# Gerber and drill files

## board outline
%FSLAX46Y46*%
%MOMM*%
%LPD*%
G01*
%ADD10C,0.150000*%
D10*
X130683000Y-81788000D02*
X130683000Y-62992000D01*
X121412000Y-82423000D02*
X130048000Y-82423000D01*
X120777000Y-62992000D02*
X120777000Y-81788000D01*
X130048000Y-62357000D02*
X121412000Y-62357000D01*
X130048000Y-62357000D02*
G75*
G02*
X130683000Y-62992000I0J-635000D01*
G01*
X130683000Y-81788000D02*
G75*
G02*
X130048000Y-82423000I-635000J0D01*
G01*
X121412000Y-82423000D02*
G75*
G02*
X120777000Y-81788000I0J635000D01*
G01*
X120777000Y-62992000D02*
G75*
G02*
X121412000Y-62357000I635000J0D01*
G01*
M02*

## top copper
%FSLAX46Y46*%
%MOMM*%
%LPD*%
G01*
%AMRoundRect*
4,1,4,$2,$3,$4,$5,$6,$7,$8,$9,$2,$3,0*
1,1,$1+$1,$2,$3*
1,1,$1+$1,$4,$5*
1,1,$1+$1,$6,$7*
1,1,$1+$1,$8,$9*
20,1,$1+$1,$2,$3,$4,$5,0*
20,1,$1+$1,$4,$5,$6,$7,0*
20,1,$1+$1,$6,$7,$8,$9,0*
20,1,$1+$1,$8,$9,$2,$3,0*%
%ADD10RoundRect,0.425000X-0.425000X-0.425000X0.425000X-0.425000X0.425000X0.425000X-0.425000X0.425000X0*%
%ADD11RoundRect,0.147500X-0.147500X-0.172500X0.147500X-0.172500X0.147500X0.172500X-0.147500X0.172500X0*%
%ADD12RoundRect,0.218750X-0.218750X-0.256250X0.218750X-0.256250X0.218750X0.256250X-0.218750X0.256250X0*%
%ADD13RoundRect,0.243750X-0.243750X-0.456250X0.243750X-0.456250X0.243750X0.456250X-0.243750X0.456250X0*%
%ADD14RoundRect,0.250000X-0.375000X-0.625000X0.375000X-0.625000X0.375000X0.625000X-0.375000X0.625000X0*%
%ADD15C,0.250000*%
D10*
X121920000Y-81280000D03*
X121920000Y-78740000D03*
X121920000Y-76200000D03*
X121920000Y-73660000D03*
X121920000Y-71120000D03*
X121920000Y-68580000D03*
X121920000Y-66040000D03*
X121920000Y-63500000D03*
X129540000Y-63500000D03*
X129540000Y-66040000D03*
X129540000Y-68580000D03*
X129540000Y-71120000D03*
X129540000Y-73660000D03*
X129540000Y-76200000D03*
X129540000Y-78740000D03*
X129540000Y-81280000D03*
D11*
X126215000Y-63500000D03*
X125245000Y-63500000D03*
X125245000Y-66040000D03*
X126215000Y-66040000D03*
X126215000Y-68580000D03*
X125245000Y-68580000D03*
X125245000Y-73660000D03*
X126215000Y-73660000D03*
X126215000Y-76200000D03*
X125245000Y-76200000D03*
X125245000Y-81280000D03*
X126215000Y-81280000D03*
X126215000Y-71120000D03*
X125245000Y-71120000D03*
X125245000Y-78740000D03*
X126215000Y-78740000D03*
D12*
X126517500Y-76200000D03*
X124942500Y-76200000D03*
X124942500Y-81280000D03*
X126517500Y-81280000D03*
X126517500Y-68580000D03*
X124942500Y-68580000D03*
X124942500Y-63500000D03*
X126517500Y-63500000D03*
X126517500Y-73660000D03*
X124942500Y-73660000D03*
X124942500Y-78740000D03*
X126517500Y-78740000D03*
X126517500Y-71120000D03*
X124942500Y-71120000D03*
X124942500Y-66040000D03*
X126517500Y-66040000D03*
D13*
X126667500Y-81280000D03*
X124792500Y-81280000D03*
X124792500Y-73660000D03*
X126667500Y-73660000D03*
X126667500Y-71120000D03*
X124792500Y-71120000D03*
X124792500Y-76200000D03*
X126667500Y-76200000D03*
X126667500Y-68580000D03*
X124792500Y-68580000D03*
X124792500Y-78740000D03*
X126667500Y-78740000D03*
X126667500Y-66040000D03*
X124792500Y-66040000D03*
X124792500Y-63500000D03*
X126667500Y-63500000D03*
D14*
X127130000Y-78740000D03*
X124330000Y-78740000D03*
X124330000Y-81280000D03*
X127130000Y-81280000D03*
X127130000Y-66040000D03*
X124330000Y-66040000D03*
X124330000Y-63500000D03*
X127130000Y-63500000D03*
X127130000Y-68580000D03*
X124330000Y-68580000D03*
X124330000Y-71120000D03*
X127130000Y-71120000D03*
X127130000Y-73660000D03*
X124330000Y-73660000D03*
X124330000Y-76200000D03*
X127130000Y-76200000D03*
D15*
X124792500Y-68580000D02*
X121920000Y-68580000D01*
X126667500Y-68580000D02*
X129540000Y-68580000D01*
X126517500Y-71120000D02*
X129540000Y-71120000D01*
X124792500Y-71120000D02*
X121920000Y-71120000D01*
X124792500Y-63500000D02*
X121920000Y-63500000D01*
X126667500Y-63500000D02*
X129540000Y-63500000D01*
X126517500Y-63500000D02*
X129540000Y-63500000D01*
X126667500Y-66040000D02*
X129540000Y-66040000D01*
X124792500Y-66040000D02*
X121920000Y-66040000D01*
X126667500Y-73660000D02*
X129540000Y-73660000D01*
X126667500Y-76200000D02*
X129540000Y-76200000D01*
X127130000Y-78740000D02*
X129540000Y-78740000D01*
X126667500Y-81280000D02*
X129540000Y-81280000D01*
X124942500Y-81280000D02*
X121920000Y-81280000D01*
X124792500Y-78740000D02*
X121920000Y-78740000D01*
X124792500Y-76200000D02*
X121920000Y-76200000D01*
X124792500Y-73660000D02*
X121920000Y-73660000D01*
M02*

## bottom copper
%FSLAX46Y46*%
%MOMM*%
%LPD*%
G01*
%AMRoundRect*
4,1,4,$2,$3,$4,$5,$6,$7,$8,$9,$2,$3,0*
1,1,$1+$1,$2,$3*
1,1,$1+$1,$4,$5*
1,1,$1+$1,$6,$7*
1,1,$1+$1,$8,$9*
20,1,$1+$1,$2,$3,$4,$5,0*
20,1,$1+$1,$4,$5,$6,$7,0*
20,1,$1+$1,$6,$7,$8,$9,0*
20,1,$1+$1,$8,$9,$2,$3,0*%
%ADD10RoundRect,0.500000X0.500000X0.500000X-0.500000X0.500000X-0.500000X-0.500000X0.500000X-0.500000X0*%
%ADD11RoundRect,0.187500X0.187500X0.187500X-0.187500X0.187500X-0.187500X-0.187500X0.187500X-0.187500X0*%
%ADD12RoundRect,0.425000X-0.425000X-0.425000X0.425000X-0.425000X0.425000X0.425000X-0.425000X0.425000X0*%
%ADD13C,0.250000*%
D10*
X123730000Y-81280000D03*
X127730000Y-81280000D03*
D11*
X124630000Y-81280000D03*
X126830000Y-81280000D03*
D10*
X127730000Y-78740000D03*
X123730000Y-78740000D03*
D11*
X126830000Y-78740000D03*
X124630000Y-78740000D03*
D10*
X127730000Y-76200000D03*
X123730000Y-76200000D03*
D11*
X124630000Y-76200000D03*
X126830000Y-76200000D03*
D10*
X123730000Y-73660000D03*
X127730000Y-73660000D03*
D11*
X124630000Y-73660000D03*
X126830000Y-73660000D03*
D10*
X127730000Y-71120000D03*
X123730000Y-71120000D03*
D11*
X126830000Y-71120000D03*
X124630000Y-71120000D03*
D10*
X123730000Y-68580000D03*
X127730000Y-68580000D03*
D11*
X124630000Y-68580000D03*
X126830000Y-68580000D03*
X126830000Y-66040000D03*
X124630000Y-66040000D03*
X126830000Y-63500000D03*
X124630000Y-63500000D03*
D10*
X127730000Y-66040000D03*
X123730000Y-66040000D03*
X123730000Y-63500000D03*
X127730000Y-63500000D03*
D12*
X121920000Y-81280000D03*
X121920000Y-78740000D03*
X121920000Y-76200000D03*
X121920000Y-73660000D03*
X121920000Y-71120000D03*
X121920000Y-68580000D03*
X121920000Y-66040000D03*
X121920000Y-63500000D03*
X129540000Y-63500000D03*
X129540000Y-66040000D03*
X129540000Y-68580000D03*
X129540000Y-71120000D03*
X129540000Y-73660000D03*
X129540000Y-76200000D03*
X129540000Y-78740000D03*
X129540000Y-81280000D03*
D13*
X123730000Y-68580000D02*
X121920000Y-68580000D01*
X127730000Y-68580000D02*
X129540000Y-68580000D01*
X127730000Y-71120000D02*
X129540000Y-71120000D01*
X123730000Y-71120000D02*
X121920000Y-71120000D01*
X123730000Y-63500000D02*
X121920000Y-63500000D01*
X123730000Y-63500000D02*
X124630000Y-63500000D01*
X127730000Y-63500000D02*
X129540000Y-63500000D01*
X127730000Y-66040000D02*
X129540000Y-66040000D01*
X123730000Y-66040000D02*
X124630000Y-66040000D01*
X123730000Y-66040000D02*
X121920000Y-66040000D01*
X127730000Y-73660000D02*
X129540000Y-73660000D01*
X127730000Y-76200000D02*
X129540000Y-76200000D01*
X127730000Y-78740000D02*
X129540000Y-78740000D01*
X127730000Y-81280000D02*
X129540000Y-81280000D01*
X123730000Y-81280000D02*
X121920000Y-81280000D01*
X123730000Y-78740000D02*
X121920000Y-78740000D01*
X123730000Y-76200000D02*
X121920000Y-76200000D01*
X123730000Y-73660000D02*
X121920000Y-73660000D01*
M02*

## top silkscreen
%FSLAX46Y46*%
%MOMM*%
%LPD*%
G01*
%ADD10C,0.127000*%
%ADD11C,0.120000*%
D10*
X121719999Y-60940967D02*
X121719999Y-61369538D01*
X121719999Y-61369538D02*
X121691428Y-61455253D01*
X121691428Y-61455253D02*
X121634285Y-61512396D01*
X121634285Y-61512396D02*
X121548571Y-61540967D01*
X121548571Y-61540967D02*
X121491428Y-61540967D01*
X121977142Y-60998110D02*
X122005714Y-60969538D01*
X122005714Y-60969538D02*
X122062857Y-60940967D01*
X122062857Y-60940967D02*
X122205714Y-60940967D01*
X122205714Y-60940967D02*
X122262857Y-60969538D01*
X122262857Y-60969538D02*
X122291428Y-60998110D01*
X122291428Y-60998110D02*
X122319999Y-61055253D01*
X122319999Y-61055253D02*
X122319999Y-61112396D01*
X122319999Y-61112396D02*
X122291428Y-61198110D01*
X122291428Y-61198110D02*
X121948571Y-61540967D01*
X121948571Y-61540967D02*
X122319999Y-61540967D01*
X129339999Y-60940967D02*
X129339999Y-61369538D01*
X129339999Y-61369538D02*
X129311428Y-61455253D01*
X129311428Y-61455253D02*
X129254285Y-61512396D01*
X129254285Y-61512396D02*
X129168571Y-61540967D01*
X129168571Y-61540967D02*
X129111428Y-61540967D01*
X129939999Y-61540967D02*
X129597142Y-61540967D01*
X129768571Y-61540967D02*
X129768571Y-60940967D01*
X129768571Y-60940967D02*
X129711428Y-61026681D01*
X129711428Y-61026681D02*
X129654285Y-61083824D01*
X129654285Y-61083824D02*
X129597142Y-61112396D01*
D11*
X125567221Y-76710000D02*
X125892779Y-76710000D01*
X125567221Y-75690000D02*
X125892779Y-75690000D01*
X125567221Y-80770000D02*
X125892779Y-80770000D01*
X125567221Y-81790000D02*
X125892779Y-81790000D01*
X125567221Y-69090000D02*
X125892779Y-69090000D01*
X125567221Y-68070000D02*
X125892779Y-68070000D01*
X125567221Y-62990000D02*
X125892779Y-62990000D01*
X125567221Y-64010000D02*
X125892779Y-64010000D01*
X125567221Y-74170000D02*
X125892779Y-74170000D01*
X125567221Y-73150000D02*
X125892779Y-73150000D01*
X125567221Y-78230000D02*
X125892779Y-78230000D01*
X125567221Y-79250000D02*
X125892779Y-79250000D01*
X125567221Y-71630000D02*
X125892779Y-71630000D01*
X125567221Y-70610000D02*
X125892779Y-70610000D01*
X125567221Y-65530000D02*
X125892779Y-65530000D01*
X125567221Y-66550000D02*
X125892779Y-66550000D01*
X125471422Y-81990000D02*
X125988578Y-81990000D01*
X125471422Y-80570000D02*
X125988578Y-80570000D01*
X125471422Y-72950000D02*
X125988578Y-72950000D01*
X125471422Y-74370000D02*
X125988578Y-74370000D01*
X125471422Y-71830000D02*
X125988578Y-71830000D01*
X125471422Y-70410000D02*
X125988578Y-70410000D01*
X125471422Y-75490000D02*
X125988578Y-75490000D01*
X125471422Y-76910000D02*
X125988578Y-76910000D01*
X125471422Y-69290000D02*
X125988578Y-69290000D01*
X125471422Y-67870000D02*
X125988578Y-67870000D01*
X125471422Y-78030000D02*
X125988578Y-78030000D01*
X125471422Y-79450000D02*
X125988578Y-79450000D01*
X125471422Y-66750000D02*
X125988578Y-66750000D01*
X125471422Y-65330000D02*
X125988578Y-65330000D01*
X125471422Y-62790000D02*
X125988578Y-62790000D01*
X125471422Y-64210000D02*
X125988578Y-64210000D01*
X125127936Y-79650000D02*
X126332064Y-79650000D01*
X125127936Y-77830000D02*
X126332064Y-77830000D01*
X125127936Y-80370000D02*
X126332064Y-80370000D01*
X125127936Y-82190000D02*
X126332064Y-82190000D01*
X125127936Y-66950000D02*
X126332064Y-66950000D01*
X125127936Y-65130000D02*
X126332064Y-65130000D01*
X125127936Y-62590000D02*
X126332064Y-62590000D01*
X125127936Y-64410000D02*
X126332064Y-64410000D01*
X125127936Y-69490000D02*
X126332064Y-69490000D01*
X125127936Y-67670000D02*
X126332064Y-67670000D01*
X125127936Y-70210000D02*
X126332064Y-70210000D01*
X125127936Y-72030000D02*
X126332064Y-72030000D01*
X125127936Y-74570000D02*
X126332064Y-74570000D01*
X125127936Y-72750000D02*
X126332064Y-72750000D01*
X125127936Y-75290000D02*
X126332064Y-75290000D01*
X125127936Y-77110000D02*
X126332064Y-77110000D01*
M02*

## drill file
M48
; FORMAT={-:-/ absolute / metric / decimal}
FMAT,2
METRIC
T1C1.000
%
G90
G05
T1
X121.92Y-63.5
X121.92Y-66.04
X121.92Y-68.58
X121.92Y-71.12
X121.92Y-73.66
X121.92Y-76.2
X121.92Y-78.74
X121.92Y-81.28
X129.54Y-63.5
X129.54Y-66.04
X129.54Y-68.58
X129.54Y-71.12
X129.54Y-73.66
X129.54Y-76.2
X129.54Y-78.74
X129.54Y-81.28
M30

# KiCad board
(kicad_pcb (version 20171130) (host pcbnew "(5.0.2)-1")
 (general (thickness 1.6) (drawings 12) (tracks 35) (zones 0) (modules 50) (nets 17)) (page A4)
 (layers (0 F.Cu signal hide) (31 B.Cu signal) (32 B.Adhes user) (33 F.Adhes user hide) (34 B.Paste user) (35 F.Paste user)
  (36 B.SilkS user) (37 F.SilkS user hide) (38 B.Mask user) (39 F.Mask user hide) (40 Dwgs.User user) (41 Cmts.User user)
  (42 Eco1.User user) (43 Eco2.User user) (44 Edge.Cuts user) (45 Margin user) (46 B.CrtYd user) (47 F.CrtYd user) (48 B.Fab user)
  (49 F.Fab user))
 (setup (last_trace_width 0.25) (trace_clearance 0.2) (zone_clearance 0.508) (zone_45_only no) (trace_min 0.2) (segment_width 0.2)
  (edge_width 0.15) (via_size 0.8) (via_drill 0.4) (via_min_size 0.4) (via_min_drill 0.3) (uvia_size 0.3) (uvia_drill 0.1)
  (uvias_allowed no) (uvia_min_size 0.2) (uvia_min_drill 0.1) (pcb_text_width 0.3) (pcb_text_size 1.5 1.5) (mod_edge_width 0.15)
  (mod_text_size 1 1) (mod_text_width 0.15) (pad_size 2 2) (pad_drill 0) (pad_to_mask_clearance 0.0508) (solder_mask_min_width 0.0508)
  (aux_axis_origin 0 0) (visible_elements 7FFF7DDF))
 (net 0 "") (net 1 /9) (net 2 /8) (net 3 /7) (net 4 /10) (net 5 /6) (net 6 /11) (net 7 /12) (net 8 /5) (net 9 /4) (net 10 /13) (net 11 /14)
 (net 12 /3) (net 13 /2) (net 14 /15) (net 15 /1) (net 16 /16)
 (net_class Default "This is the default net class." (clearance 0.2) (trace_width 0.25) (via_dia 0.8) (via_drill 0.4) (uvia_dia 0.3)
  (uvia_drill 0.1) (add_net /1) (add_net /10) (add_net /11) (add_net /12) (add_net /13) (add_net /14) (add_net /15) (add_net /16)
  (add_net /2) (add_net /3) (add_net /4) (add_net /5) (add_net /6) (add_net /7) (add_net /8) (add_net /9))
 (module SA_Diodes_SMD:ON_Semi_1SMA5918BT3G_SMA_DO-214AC (layer B.Cu) (at 125.73 81.28 180)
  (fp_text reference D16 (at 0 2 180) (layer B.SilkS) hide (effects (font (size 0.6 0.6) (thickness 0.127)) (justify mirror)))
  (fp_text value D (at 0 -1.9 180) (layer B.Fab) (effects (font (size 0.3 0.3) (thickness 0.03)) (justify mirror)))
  (pad 2 smd roundrect (at 2 0 180) (size 2 2) (layers B.Cu B.Paste B.Mask) (roundrect_rratio 0.25) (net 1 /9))
  (pad 1 smd roundrect (at -2 0 180) (size 2 2) (layers B.Cu B.Paste B.Mask) (roundrect_rratio 0.25) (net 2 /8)))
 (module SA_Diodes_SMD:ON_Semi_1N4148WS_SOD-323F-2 (layer B.Cu) (at 125.73 81.28 180)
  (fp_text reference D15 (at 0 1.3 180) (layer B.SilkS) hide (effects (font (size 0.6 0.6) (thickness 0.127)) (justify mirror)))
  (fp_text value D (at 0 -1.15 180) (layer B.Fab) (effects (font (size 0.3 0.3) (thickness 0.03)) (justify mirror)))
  (pad 2 smd roundrect (at 1.1 0 180) (size 0.75 0.75) (layers B.Cu B.Paste B.Mask) (roundrect_rratio 0.25) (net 1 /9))
  (pad 1 smd roundrect (at -1.1 0 180) (size 0.75 0.75) (layers B.Cu B.Paste B.Mask) (roundrect_rratio 0.25) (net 2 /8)))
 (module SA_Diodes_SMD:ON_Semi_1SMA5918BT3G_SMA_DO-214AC (layer B.Cu) (at 125.73 78.74 180)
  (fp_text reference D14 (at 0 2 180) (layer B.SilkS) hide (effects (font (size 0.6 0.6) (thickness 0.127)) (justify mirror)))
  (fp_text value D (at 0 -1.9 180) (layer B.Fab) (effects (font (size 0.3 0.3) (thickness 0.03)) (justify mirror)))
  (pad 1 smd roundrect (at -2 0 180) (size 2 2) (layers B.Cu B.Paste B.Mask) (roundrect_rratio 0.25) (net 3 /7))
  (pad 2 smd roundrect (at 2 0 180) (size 2 2) (layers B.Cu B.Paste B.Mask) (roundrect_rratio 0.25) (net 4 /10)))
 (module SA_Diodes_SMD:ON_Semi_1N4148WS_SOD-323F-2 (layer B.Cu) (at 125.73 78.74 180)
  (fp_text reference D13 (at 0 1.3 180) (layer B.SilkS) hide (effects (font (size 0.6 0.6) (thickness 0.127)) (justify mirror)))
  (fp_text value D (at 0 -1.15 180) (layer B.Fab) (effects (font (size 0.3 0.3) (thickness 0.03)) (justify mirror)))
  (pad 1 smd roundrect (at -1.1 0 180) (size 0.75 0.75) (layers B.Cu B.Paste B.Mask) (roundrect_rratio 0.25) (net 3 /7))
  (pad 2 smd roundrect (at 1.1 0 180) (size 0.75 0.75) (layers B.Cu B.Paste B.Mask) (roundrect_rratio 0.25) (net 4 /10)))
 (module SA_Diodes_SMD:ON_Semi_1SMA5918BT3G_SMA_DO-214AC (layer B.Cu) (at 125.73 76.2 180)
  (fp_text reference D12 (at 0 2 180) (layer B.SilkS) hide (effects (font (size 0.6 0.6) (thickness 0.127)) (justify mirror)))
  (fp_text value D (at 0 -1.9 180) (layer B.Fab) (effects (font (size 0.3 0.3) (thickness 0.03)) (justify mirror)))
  (pad 1 smd roundrect (at -2 0 180) (size 2 2) (layers B.Cu B.Paste B.Mask) (roundrect_rratio 0.25) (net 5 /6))
  (pad 2 smd roundrect (at 2 0 180) (size 2 2) (layers B.Cu B.Paste B.Mask) (roundrect_rratio 0.25) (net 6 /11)))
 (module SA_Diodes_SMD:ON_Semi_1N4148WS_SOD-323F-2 (layer B.Cu) (at 125.73 76.2 180)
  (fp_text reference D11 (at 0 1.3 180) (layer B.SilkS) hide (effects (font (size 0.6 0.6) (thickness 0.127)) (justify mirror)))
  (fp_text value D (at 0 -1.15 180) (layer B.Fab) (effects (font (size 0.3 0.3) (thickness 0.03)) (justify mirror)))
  (pad 2 smd roundrect (at 1.1 0 180) (size 0.75 0.75) (layers B.Cu B.Paste B.Mask) (roundrect_rratio 0.25) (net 6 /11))
  (pad 1 smd roundrect (at -1.1 0 180) (size 0.75 0.75) (layers B.Cu B.Paste B.Mask) (roundrect_rratio 0.25) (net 5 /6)))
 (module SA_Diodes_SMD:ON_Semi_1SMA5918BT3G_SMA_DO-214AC (layer B.Cu) (at 125.73 73.66 180)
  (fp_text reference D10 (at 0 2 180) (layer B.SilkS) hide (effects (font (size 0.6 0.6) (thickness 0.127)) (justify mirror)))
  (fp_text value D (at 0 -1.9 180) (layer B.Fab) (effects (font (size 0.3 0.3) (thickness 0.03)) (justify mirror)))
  (pad 2 smd roundrect (at 2 0 180) (size 2 2) (layers B.Cu B.Paste B.Mask) (roundrect_rratio 0.25) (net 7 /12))
  (pad 1 smd roundrect (at -2 0 180) (size 2 2) (layers B.Cu B.Paste B.Mask) (roundrect_rratio 0.25) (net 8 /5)))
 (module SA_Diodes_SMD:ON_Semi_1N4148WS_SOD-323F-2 (layer B.Cu) (at 125.73 73.66 180)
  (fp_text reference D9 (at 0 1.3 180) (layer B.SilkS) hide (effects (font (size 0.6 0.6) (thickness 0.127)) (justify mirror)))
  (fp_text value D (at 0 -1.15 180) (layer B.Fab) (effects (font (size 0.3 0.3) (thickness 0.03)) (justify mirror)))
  (pad 2 smd roundrect (at 1.1 0 180) (size 0.75 0.75) (layers B.Cu B.Paste B.Mask) (roundrect_rratio 0.25) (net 7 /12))
  (pad 1 smd roundrect (at -1.1 0 180) (size 0.75 0.75) (layers B.Cu B.Paste B.Mask) (roundrect_rratio 0.25) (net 8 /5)))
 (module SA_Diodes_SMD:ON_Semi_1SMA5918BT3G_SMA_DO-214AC (layer B.Cu) (at 125.73 71.12 180)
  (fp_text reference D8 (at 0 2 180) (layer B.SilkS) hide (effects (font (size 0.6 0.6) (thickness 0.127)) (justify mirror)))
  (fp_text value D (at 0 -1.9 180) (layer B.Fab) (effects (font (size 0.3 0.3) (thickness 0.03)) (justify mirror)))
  (pad 1 smd roundrect (at -2 0 180) (size 2 2) (layers B.Cu B.Paste B.Mask) (roundrect_rratio 0.25) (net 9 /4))
  (pad 2 smd roundrect (at 2 0 180) (size 2 2) (layers B.Cu B.Paste B.Mask) (roundrect_rratio 0.25) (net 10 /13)))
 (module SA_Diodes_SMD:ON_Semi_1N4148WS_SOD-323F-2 (layer B.Cu) (at 125.73 71.12 180)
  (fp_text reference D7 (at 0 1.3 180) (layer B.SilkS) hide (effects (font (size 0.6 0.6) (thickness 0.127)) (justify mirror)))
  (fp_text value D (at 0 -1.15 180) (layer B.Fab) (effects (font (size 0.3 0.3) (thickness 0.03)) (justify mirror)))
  (pad 1 smd roundrect (at -1.1 0 180) (size 0.75 0.75) (layers B.Cu B.Paste B.Mask) (roundrect_rratio 0.25) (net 9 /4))
  (pad 2 smd roundrect (at 1.1 0 180) (size 0.75 0.75) (layers B.Cu B.Paste B.Mask) (roundrect_rratio 0.25) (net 10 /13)))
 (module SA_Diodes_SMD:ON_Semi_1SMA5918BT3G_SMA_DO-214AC (layer B.Cu) (at 125.73 68.58 180)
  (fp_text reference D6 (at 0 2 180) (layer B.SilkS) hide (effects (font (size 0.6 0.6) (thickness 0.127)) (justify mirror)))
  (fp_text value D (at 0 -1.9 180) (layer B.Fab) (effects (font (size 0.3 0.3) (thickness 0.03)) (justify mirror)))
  (pad 2 smd roundrect (at 2 0 180) (size 2 2) (layers B.Cu B.Paste B.Mask) (roundrect_rratio 0.25) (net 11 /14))
  (pad 1 smd roundrect (at -2 0 180) (size 2 2) (layers B.Cu B.Paste B.Mask) (roundrect_rratio 0.25) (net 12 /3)))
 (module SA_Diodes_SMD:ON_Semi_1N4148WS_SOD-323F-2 (layer B.Cu) (at 125.73 68.58 180)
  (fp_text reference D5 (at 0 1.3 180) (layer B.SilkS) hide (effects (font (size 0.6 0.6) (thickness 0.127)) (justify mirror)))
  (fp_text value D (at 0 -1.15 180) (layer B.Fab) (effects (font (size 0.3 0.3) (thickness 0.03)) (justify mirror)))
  (pad 2 smd roundrect (at 1.1 0 180) (size 0.75 0.75) (layers B.Cu B.Paste B.Mask) (roundrect_rratio 0.25) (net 11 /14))
  (pad 1 smd roundrect (at -1.1 0 180) (size 0.75 0.75) (layers B.Cu B.Paste B.Mask) (roundrect_rratio 0.25) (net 12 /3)))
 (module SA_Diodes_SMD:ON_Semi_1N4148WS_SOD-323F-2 (layer B.Cu) (at 125.73 66.04 180)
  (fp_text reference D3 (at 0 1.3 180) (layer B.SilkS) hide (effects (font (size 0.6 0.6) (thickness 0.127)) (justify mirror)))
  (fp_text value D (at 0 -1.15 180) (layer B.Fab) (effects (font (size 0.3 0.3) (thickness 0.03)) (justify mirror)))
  (pad 1 smd roundrect (at -1.1 0 180) (size 0.75 0.75) (layers B.Cu B.Paste B.Mask) (roundrect_rratio 0.25) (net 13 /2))
  (pad 2 smd roundrect (at 1.1 0 180) (size 0.75 0.75) (layers B.Cu B.Paste B.Mask) (roundrect_rratio 0.25) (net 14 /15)))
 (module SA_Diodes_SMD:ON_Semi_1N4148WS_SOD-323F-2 (layer B.Cu) (at 125.73 63.5 180)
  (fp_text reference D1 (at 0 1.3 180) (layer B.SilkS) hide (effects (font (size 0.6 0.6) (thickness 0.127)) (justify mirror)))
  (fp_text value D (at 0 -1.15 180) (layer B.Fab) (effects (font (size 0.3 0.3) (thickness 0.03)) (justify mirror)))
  (pad 1 smd roundrect (at -1.1 0 180) (size 0.75 0.75) (layers B.Cu B.Paste B.Mask) (roundrect_rratio 0.25) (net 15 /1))
  (pad 2 smd roundrect (at 1.1 0 180) (size 0.75 0.75) (layers B.Cu B.Paste B.Mask) (roundrect_rratio 0.25) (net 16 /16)))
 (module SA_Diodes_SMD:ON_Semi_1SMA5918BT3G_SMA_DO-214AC (layer B.Cu) (at 125.73 66.04 180)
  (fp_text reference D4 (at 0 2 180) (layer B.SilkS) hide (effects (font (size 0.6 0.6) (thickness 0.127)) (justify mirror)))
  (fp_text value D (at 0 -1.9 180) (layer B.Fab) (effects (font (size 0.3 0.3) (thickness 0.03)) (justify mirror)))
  (pad 1 smd roundrect (at -2 0 180) (size 2 2) (layers B.Cu B.Paste B.Mask) (roundrect_rratio 0.25) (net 13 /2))
  (pad 2 smd roundrect (at 2 0 180) (size 2 2) (layers B.Cu B.Paste B.Mask) (roundrect_rratio 0.25) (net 14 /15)))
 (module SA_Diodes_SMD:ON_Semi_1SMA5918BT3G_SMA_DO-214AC (layer B.Cu) (at 125.73 63.5 180)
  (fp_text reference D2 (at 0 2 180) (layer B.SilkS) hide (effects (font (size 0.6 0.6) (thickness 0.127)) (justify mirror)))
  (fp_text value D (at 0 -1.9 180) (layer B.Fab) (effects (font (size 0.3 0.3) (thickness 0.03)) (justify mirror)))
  (pad 2 smd roundrect (at 2 0 180) (size 2 2) (layers B.Cu B.Paste B.Mask) (roundrect_rratio 0.25) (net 16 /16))
  (pad 1 smd roundrect (at -2 0 180) (size 2 2) (layers B.Cu B.Paste B.Mask) (roundrect_rratio 0.25) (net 15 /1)))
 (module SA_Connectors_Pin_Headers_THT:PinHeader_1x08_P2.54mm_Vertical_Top (layer F.Cu) (at 121.92 63.5)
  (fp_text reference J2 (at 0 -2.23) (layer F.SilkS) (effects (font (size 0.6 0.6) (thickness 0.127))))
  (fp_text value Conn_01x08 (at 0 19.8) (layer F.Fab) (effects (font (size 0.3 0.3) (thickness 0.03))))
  (pad 8 thru_hole roundrect (at 0 17.78) (size 1.7 1.7) (drill 1) (layers *.Cu *.Mask) (roundrect_rratio 0.25) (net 1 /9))
  (pad 7 thru_hole roundrect (at 0 15.24) (size 1.7 1.7) (drill 1) (layers *.Cu *.Mask) (roundrect_rratio 0.25) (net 4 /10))
  (pad 6 thru_hole roundrect (at 0 12.7) (size 1.7 1.7) (drill 1) (layers *.Cu *.Mask) (roundrect_rratio 0.25) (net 6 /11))
  (pad 5 thru_hole roundrect (at 0 10.16) (size 1.7 1.7) (drill 1) (layers *.Cu *.Mask) (roundrect_rratio 0.25) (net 7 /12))
  (pad 4 thru_hole roundrect (at 0 7.62) (size 1.7 1.7) (drill 1) (layers *.Cu *.Mask) (roundrect_rratio 0.25) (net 10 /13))
  (pad 3 thru_hole roundrect (at 0 5.08) (size 1.7 1.7) (drill 1) (layers *.Cu *.Mask) (roundrect_rratio 0.25) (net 11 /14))
  (pad 2 thru_hole roundrect (at 0 2.54) (size 1.7 1.7) (drill 1) (layers *.Cu *.Mask) (roundrect_rratio 0.25) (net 14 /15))
  (pad 1 thru_hole roundrect (at 0 0) (size 1.7 1.7) (drill 1) (layers *.Cu *.Mask) (roundrect_rratio 0.25) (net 16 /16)))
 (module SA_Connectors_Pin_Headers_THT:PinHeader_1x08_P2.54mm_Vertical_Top (layer F.Cu) (at 129.54 63.5)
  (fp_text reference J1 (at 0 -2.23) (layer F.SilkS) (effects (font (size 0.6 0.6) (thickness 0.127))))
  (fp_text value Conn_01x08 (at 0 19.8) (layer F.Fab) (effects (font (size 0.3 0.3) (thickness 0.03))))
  (pad 1 thru_hole roundrect (at 0 0) (size 1.7 1.7) (drill 1) (layers *.Cu *.Mask) (roundrect_rratio 0.25) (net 15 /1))
  (pad 2 thru_hole roundrect (at 0 2.54) (size 1.7 1.7) (drill 1) (layers *.Cu *.Mask) (roundrect_rratio 0.25) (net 13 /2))
  (pad 3 thru_hole roundrect (at 0 5.08) (size 1.7 1.7) (drill 1) (layers *.Cu *.Mask) (roundrect_rratio 0.25) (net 12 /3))
  (pad 4 thru_hole roundrect (at 0 7.62) (size 1.7 1.7) (drill 1) (layers *.Cu *.Mask) (roundrect_rratio 0.25) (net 9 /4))
  (pad 5 thru_hole roundrect (at 0 10.16) (size 1.7 1.7) (drill 1) (layers *.Cu *.Mask) (roundrect_rratio 0.25) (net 8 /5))
  (pad 6 thru_hole roundrect (at 0 12.7) (size 1.7 1.7) (drill 1) (layers *.Cu *.Mask) (roundrect_rratio 0.25) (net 5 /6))
  (pad 7 thru_hole roundrect (at 0 15.24) (size 1.7 1.7) (drill 1) (layers *.Cu *.Mask) (roundrect_rratio 0.25) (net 3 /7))
  (pad 8 thru_hole roundrect (at 0 17.78) (size 1.7 1.7) (drill 1) (layers *.Cu *.Mask) (roundrect_rratio 0.25) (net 2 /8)))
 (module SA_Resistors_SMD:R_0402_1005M (layer F.Cu) (at 125.73 63.5)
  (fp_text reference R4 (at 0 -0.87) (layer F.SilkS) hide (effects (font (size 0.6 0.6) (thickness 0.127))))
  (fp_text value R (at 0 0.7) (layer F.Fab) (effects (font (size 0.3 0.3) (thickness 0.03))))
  (pad 2 smd roundrect (at 0.485 0) (size 0.59 0.64) (layers F.Cu F.Paste F.Mask) (roundrect_rratio 0.25) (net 15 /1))
  (pad 1 smd roundrect (at -0.485 0) (size 0.59 0.64) (layers F.Cu F.Paste F.Mask) (roundrect_rratio 0.25) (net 16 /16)))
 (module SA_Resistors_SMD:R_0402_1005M (layer F.Cu) (at 125.73 66.04)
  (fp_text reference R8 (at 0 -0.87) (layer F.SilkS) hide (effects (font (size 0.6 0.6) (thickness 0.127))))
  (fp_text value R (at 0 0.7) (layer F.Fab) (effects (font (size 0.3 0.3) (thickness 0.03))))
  (pad 1 smd roundrect (at -0.485 0) (size 0.59 0.64) (layers F.Cu F.Paste F.Mask) (roundrect_rratio 0.25) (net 14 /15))
  (pad 2 smd roundrect (at 0.485 0) (size 0.59 0.64) (layers F.Cu F.Paste F.Mask) (roundrect_rratio 0.25) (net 13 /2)))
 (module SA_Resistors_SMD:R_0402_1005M (layer F.Cu) (at 125.73 68.58)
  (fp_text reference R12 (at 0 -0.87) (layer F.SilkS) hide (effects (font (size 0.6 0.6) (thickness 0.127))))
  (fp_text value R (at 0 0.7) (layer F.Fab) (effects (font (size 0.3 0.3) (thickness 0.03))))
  (pad 2 smd roundrect (at 0.485 0) (size 0.59 0.64) (layers F.Cu F.Paste F.Mask) (roundrect_rratio 0.25) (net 12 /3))
  (pad 1 smd roundrect (at -0.485 0) (size 0.59 0.64) (layers F.Cu F.Paste F.Mask) (roundrect_rratio 0.25) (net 11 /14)))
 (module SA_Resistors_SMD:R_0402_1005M (layer F.Cu) (at 125.73 73.66)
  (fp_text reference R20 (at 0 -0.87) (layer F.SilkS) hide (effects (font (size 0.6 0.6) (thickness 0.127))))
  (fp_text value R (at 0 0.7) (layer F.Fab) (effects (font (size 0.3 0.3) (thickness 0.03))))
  (pad 1 smd roundrect (at -0.485 0) (size 0.59 0.64) (layers F.Cu F.Paste F.Mask) (roundrect_rratio 0.25) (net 7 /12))
  (pad 2 smd roundrect (at 0.485 0) (size 0.59 0.64) (layers F.Cu F.Paste F.Mask) (roundrect_rratio 0.25) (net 8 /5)))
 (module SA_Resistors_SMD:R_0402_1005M (layer F.Cu) (at 125.73 76.2)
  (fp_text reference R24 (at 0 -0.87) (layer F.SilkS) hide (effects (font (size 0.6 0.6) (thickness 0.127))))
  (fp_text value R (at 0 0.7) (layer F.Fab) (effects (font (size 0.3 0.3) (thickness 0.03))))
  (pad 2 smd roundrect (at 0.485 0) (size 0.59 0.64) (layers F.Cu F.Paste F.Mask) (roundrect_rratio 0.25) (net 5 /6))
  (pad 1 smd roundrect (at -0.485 0) (size 0.59 0.64) (layers F.Cu F.Paste F.Mask) (roundrect_rratio 0.25) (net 6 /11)))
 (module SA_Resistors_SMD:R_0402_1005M (layer F.Cu) (at 125.73 81.28)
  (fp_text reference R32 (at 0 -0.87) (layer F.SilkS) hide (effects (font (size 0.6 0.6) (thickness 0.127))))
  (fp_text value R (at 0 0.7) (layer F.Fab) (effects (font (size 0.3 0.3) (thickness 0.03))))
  (pad 1 smd roundrect (at -0.485 0) (size 0.59 0.64) (layers F.Cu F.Paste F.Mask) (roundrect_rratio 0.25) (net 1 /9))
  (pad 2 smd roundrect (at 0.485 0) (size 0.59 0.64) (layers F.Cu F.Paste F.Mask) (roundrect_rratio 0.25) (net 2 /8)))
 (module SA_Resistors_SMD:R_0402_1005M (layer F.Cu) (at 125.73 71.12)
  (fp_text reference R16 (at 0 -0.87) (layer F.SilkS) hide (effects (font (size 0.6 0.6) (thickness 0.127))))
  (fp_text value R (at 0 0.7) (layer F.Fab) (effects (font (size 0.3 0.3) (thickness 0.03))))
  (pad 2 smd roundrect (at 0.485 0) (size 0.59 0.64) (layers F.Cu F.Paste F.Mask) (roundrect_rratio 0.25) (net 9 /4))
  (pad 1 smd roundrect (at -0.485 0) (size 0.59 0.64) (layers F.Cu F.Paste F.Mask) (roundrect_rratio 0.25) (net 10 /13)))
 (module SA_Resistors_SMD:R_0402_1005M (layer F.Cu) (at 125.73 78.74)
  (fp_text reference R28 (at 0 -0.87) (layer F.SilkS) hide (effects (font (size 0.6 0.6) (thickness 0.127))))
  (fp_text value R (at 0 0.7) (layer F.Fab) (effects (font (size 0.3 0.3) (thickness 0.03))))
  (pad 1 smd roundrect (at -0.485 0) (size 0.59 0.64) (layers F.Cu F.Paste F.Mask) (roundrect_rratio 0.25) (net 4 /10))
  (pad 2 smd roundrect (at 0.485 0) (size 0.59 0.64) (layers F.Cu F.Paste F.Mask) (roundrect_rratio 0.25) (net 3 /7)))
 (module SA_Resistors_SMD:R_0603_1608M (layer F.Cu) (at 125.73 76.2)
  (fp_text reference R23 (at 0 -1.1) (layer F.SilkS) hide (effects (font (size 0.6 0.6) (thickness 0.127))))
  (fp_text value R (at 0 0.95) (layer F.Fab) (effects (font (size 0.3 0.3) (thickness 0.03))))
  (fp_line (start -0.162779 0.51) (end 0.162779 0.51) (layer F.SilkS) (width 0.12))
  (fp_line (start -0.162779 -0.51) (end 0.162779 -0.51) (layer F.SilkS) (width 0.12))
  (pad 2 smd roundrect (at 0.7875 0) (size 0.875 0.95) (layers F.Cu F.Paste F.Mask) (roundrect_rratio 0.25) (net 5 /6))
  (pad 1 smd roundrect (at -0.7875 0) (size 0.875 0.95) (layers F.Cu F.Paste F.Mask) (roundrect_rratio 0.25) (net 6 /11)))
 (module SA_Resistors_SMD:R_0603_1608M (layer F.Cu) (at 125.73 81.28)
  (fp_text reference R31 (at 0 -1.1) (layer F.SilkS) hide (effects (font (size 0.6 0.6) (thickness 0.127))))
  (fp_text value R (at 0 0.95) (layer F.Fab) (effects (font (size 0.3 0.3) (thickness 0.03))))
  (fp_line (start -0.162779 -0.51) (end 0.162779 -0.51) (layer F.SilkS) (width 0.12))
  (fp_line (start -0.162779 0.51) (end 0.162779 0.51) (layer F.SilkS) (width 0.12))
  (pad 1 smd roundrect (at -0.7875 0) (size 0.875 0.95) (layers F.Cu F.Paste F.Mask) (roundrect_rratio 0.25) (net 1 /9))
  (pad 2 smd roundrect (at 0.7875 0) (size 0.875 0.95) (layers F.Cu F.Paste F.Mask) (roundrect_rratio 0.25) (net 2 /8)))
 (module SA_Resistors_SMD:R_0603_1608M (layer F.Cu) (at 125.73 68.58)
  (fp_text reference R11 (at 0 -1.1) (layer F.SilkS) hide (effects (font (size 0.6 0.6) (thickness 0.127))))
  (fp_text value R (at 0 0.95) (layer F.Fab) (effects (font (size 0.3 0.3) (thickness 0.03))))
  (fp_line (start -0.162779 0.51) (end 0.162779 0.51) (layer F.SilkS) (width 0.12))
  (fp_line (start -0.162779 -0.51) (end 0.162779 -0.51) (layer F.SilkS) (width 0.12))
  (pad 2 smd roundrect (at 0.7875 0) (size 0.875 0.95) (layers F.Cu F.Paste F.Mask) (roundrect_rratio 0.25) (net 12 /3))
  (pad 1 smd roundrect (at -0.7875 0) (size 0.875 0.95) (layers F.Cu F.Paste F.Mask) (roundrect_rratio 0.25) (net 11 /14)))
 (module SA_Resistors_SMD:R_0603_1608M (layer F.Cu) (at 125.73 63.5)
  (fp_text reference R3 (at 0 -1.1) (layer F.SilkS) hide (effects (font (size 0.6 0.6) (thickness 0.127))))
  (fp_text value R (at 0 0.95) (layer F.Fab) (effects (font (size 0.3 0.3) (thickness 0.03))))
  (fp_line (start -0.162779 -0.51) (end 0.162779 -0.51) (layer F.SilkS) (width 0.12))
  (fp_line (start -0.162779 0.51) (end 0.162779 0.51) (layer F.SilkS) (width 0.12))
  (pad 1 smd roundrect (at -0.7875 0) (size 0.875 0.95) (layers F.Cu F.Paste F.Mask) (roundrect_rratio 0.25) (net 16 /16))
  (pad 2 smd roundrect (at 0.7875 0) (size 0.875 0.95) (layers F.Cu F.Paste F.Mask) (roundrect_rratio 0.25) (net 15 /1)))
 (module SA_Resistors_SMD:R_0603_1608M (layer F.Cu) (at 125.73 73.66)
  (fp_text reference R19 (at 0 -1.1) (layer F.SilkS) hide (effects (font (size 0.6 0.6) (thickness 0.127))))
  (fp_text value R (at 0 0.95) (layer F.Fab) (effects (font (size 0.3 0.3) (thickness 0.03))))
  (fp_line (start -0.162779 0.51) (end 0.162779 0.51) (layer F.SilkS) (width 0.12))
  (fp_line (start -0.162779 -0.51) (end 0.162779 -0.51) (layer F.SilkS) (width 0.12))
  (pad 2 smd roundrect (at 0.7875 0) (size 0.875 0.95) (layers F.Cu F.Paste F.Mask) (roundrect_rratio 0.25) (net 8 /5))
  (pad 1 smd roundrect (at -0.7875 0) (size 0.875 0.95) (layers F.Cu F.Paste F.Mask) (roundrect_rratio 0.25) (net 7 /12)))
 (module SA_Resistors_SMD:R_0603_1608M (layer F.Cu) (at 125.73 78.74)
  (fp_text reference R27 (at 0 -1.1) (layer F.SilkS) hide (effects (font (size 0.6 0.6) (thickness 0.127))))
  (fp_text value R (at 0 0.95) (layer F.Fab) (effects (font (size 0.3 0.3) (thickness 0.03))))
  (fp_line (start -0.162779 -0.51) (end 0.162779 -0.51) (layer F.SilkS) (width 0.12))
  (fp_line (start -0.162779 0.51) (end 0.162779 0.51) (layer F.SilkS) (width 0.12))
  (pad 1 smd roundrect (at -0.7875 0) (size 0.875 0.95) (layers F.Cu F.Paste F.Mask) (roundrect_rratio 0.25) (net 4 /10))
  (pad 2 smd roundrect (at 0.7875 0) (size 0.875 0.95) (layers F.Cu F.Paste F.Mask) (roundrect_rratio 0.25) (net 3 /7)))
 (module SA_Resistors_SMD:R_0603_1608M (layer F.Cu) (at 125.73 71.12)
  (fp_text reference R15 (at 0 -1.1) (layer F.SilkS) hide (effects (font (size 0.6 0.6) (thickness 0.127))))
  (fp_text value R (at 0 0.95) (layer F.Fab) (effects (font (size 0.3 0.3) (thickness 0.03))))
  (fp_line (start -0.162779 0.51) (end 0.162779 0.51) (layer F.SilkS) (width 0.12))
  (fp_line (start -0.162779 -0.51) (end 0.162779 -0.51) (layer F.SilkS) (width 0.12))
  (pad 2 smd roundrect (at 0.7875 0) (size 0.875 0.95) (layers F.Cu F.Paste F.Mask) (roundrect_rratio 0.25) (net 9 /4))
  (pad 1 smd roundrect (at -0.7875 0) (size 0.875 0.95) (layers F.Cu F.Paste F.Mask) (roundrect_rratio 0.25) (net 10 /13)))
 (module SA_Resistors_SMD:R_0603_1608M (layer F.Cu) (at 125.73 66.04)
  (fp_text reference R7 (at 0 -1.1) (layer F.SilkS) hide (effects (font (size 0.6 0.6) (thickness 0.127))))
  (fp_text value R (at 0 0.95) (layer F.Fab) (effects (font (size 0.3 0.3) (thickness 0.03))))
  (fp_line (start -0.162779 -0.51) (end 0.162779 -0.51) (layer F.SilkS) (width 0.12))
  (fp_line (start -0.162779 0.51) (end 0.162779 0.51) (layer F.SilkS) (width 0.12))
  (pad 1 smd roundrect (at -0.7875 0) (size 0.875 0.95) (layers F.Cu F.Paste F.Mask) (roundrect_rratio 0.25) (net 14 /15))
  (pad 2 smd roundrect (at 0.7875 0) (size 0.875 0.95) (layers F.Cu F.Paste F.Mask) (roundrect_rratio 0.25) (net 13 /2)))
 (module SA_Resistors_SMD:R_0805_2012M (layer F.Cu) (at 125.73 81.28)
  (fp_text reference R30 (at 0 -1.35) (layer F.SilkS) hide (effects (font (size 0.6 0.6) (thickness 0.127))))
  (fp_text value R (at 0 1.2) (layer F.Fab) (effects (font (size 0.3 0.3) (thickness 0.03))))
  (fp_line (start -0.258578 0.71) (end 0.258578 0.71) (layer F.SilkS) (width 0.12))
  (fp_line (start -0.258578 -0.71) (end 0.258578 -0.71) (layer F.SilkS) (width 0.12))
  (pad 2 smd roundrect (at 0.9375 0) (size 0.975 1.4) (layers F.Cu F.Paste F.Mask) (roundrect_rratio 0.25) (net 2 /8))
  (pad 1 smd roundrect (at -0.9375 0) (size 0.975 1.4) (layers F.Cu F.Paste F.Mask) (roundrect_rratio 0.25) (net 1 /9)))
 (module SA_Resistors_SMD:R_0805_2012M (layer F.Cu) (at 125.73 73.66)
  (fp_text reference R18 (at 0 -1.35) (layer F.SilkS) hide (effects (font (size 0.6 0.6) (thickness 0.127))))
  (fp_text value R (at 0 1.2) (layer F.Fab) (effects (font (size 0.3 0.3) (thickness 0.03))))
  (fp_line (start -0.258578 -0.71) (end 0.258578 -0.71) (layer F.SilkS) (width 0.12))
  (fp_line (start -0.258578 0.71) (end 0.258578 0.71) (layer F.SilkS) (width 0.12))
  (pad 1 smd roundrect (at -0.9375 0) (size 0.975 1.4) (layers F.Cu F.Paste F.Mask) (roundrect_rratio 0.25) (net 7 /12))
  (pad 2 smd roundrect (at 0.9375 0) (size 0.975 1.4) (layers F.Cu F.Paste F.Mask) (roundrect_rratio 0.25) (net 8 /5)))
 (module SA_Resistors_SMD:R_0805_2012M (layer F.Cu) (at 125.73 71.12)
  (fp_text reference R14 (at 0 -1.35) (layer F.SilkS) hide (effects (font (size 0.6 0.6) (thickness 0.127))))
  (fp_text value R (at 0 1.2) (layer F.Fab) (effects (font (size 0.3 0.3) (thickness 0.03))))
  (fp_line (start -0.258578 0.71) (end 0.258578 0.71) (layer F.SilkS) (width 0.12))
  (fp_line (start -0.258578 -0.71) (end 0.258578 -0.71) (layer F.SilkS) (width 0.12))
  (pad 2 smd roundrect (at 0.9375 0) (size 0.975 1.4) (layers F.Cu F.Paste F.Mask) (roundrect_rratio 0.25) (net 9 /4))
  (pad 1 smd roundrect (at -0.9375 0) (size 0.975 1.4) (layers F.Cu F.Paste F.Mask) (roundrect_rratio 0.25) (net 10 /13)))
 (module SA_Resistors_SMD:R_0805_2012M (layer F.Cu) (at 125.73 76.2)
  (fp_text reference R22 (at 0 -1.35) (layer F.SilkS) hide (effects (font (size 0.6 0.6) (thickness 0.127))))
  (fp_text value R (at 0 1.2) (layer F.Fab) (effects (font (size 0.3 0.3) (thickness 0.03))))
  (fp_line (start -0.258578 -0.71) (end 0.258578 -0.71) (layer F.SilkS) (width 0.12))
  (fp_line (start -0.258578 0.71) (end 0.258578 0.71) (layer F.SilkS) (width 0.12))
  (pad 1 smd roundrect (at -0.9375 0) (size 0.975 1.4) (layers F.Cu F.Paste F.Mask) (roundrect_rratio 0.25) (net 6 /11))
  (pad 2 smd roundrect (at 0.9375 0) (size 0.975 1.4) (layers F.Cu F.Paste F.Mask) (roundrect_rratio 0.25) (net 5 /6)))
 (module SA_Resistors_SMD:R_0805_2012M (layer F.Cu) (at 125.73 68.58)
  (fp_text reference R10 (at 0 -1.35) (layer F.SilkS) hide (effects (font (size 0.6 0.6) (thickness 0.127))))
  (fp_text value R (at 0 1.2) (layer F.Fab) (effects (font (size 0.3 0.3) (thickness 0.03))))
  (fp_line (start -0.258578 0.71) (end 0.258578 0.71) (layer F.SilkS) (width 0.12))
  (fp_line (start -0.258578 -0.71) (end 0.258578 -0.71) (layer F.SilkS) (width 0.12))
  (pad 2 smd roundrect (at 0.9375 0) (size 0.975 1.4) (layers F.Cu F.Paste F.Mask) (roundrect_rratio 0.25) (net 12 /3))
  (pad 1 smd roundrect (at -0.9375 0) (size 0.975 1.4) (layers F.Cu F.Paste F.Mask) (roundrect_rratio 0.25) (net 11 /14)))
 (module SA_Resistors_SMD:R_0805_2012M (layer F.Cu) (at 125.73 78.74)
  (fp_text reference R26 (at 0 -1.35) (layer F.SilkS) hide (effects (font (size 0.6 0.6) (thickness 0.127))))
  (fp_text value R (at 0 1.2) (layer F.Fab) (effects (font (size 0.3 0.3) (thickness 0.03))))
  (fp_line (start -0.258578 -0.71) (end 0.258578 -0.71) (layer F.SilkS) (width 0.12))
  (fp_line (start -0.258578 0.71) (end 0.258578 0.71) (layer F.SilkS) (width 0.12))
  (pad 1 smd roundrect (at -0.9375 0) (size 0.975 1.4) (layers F.Cu F.Paste F.Mask) (roundrect_rratio 0.25) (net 4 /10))
  (pad 2 smd roundrect (at 0.9375 0) (size 0.975 1.4) (layers F.Cu F.Paste F.Mask) (roundrect_rratio 0.25) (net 3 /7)))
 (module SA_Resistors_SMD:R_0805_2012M (layer F.Cu) (at 125.73 66.04)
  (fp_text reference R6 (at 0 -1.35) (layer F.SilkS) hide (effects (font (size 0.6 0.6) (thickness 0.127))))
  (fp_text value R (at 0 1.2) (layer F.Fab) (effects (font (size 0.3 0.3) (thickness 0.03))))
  (fp_line (start -0.258578 0.71) (end 0.258578 0.71) (layer F.SilkS) (width 0.12))
  (fp_line (start -0.258578 -0.71) (end 0.258578 -0.71) (layer F.SilkS) (width 0.12))
  (pad 2 smd roundrect (at 0.9375 0) (size 0.975 1.4) (layers F.Cu F.Paste F.Mask) (roundrect_rratio 0.25) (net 13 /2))
  (pad 1 smd roundrect (at -0.9375 0) (size 0.975 1.4) (layers F.Cu F.Paste F.Mask) (roundrect_rratio 0.25) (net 14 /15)))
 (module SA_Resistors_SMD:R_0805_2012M (layer F.Cu) (at 125.73 63.5)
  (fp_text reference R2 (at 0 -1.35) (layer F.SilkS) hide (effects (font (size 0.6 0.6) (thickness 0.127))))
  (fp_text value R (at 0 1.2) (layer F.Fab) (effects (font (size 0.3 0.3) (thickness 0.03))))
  (fp_line (start -0.258578 -0.71) (end 0.258578 -0.71) (layer F.SilkS) (width 0.12))
  (fp_line (start -0.258578 0.71) (end 0.258578 0.71) (layer F.SilkS) (width 0.12))
  (pad 1 smd roundrect (at -0.9375 0) (size 0.975 1.4) (layers F.Cu F.Paste F.Mask) (roundrect_rratio 0.25) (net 16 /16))
  (pad 2 smd roundrect (at 0.9375 0) (size 0.975 1.4) (layers F.Cu F.Paste F.Mask) (roundrect_rratio 0.25) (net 15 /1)))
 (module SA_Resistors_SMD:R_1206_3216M (layer F.Cu) (at 125.73 78.74)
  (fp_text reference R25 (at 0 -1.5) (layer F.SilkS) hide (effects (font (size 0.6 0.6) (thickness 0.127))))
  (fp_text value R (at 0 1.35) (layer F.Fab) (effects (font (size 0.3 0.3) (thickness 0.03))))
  (fp_line (start -0.602064 0.91) (end 0.602064 0.91) (layer F.SilkS) (width 0.12))
  (fp_line (start -0.602064 -0.91) (end 0.602064 -0.91) (layer F.SilkS) (width 0.12))
  (pad 2 smd roundrect (at 1.4 0) (size 1.25 1.75) (layers F.Cu F.Paste F.Mask) (roundrect_rratio 0.2) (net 3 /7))
  (pad 1 smd roundrect (at -1.4 0) (size 1.25 1.75) (layers F.Cu F.Paste F.Mask) (roundrect_rratio 0.2) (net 4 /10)))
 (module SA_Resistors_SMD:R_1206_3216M (layer F.Cu) (at 125.73 81.28)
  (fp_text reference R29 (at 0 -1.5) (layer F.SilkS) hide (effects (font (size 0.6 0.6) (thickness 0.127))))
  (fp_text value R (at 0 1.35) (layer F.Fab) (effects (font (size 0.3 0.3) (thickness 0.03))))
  (fp_line (start -0.602064 -0.91) (end 0.602064 -0.91) (layer F.SilkS) (width 0.12))
  (fp_line (start -0.602064 0.91) (end 0.602064 0.91) (layer F.SilkS) (width 0.12))
  (pad 1 smd roundrect (at -1.4 0) (size 1.25 1.75) (layers F.Cu F.Paste F.Mask) (roundrect_rratio 0.2) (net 1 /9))
  (pad 2 smd roundrect (at 1.4 0) (size 1.25 1.75) (layers F.Cu F.Paste F.Mask) (roundrect_rratio 0.2) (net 2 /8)))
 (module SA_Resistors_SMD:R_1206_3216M (layer F.Cu) (at 125.73 66.04)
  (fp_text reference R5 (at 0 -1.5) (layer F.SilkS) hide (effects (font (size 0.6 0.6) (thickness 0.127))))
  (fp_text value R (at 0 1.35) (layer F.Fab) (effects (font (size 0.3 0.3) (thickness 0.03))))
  (fp_line (start -0.602064 0.91) (end 0.602064 0.91) (layer F.SilkS) (width 0.12))
  (fp_line (start -0.602064 -0.91) (end 0.602064 -0.91) (layer F.SilkS) (width 0.12))
  (pad 2 smd roundrect (at 1.4 0) (size 1.25 1.75) (layers F.Cu F.Paste F.Mask) (roundrect_rratio 0.2) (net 13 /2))
  (pad 1 smd roundrect (at -1.4 0) (size 1.25 1.75) (layers F.Cu F.Paste F.Mask) (roundrect_rratio 0.2) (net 14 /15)))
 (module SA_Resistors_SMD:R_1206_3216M (layer F.Cu) (at 125.73 63.5)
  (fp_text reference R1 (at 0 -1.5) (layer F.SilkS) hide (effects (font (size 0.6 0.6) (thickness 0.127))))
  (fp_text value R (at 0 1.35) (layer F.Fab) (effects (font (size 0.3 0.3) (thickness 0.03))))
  (fp_line (start -0.602064 -0.91) (end 0.602064 -0.91) (layer F.SilkS) (width 0.12))
  (fp_line (start -0.602064 0.91) (end 0.602064 0.91) (layer F.SilkS) (width 0.12))
  (pad 1 smd roundrect (at -1.4 0) (size 1.25 1.75) (layers F.Cu F.Paste F.Mask) (roundrect_rratio 0.2) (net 16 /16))
  (pad 2 smd roundrect (at 1.4 0) (size 1.25 1.75) (layers F.Cu F.Paste F.Mask) (roundrect_rratio 0.2) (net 15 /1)))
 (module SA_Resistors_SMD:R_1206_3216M (layer F.Cu) (at 125.73 68.58)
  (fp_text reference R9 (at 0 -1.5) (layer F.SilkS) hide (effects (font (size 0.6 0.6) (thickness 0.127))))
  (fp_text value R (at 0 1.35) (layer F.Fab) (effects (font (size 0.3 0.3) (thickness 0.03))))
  (fp_line (start -0.602064 0.91) (end 0.602064 0.91) (layer F.SilkS) (width 0.12))
  (fp_line (start -0.602064 -0.91) (end 0.602064 -0.91) (layer F.SilkS) (width 0.12))
  (pad 2 smd roundrect (at 1.4 0) (size 1.25 1.75) (layers F.Cu F.Paste F.Mask) (roundrect_rratio 0.2) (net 12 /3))
  (pad 1 smd roundrect (at -1.4 0) (size 1.25 1.75) (layers F.Cu F.Paste F.Mask) (roundrect_rratio 0.2) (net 11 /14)))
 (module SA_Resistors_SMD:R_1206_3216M (layer F.Cu) (at 125.73 71.12)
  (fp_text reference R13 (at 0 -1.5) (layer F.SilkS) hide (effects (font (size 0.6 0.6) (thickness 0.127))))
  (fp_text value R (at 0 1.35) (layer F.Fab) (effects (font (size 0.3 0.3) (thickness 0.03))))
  (fp_line (start -0.602064 -0.91) (end 0.602064 -0.91) (layer F.SilkS) (width 0.12))
  (fp_line (start -0.602064 0.91) (end 0.602064 0.91) (layer F.SilkS) (width 0.12))
  (pad 1 smd roundrect (at -1.4 0) (size 1.25 1.75) (layers F.Cu F.Paste F.Mask) (roundrect_rratio 0.2) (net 10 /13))
  (pad 2 smd roundrect (at 1.4 0) (size 1.25 1.75) (layers F.Cu F.Paste F.Mask) (roundrect_rratio 0.2) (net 9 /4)))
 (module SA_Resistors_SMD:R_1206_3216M (layer F.Cu) (at 125.73 73.66)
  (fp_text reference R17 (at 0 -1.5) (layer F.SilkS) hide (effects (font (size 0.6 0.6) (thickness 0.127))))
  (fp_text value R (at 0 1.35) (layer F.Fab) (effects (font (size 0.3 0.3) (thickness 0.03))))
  (fp_line (start -0.602064 0.91) (end 0.602064 0.91) (layer F.SilkS) (width 0.12))
  (fp_line (start -0.602064 -0.91) (end 0.602064 -0.91) (layer F.SilkS) (width 0.12))
  (pad 2 smd roundrect (at 1.4 0) (size 1.25 1.75) (layers F.Cu F.Paste F.Mask) (roundrect_rratio 0.2) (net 8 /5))
  (pad 1 smd roundrect (at -1.4 0) (size 1.25 1.75) (layers F.Cu F.Paste F.Mask) (roundrect_rratio 0.2) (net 7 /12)))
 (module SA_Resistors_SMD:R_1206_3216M (layer F.Cu) (at 125.73 76.2)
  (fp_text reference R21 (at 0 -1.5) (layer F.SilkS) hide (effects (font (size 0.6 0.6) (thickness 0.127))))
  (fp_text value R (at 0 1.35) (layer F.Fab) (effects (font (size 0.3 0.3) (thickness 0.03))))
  (fp_line (start -0.602064 -0.91) (end 0.602064 -0.91) (layer F.SilkS) (width 0.12))
  (fp_line (start -0.602064 0.91) (end 0.602064 0.91) (layer F.SilkS) (width 0.12))
  (pad 1 smd roundrect (at -1.4 0) (size 1.25 1.75) (layers F.Cu F.Paste F.Mask) (roundrect_rratio 0.2) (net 6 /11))
  (pad 2 smd roundrect (at 1.4 0) (size 1.25 1.75) (layers F.Cu F.Paste F.Mask) (roundrect_rratio 0.2) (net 5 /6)))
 (gr_line (start 130.683 81.788) (end 130.683 62.992) (layer Edge.Cuts) (width 0.15))
 (gr_line (start 121.412 82.423) (end 130.048 82.423) (layer Edge.Cuts) (width 0.15))
 (gr_line (start 120.777 62.992) (end 120.777 81.788) (layer Edge.Cuts) (width 0.15))
 (gr_line (start 130.048 62.357) (end 121.412 62.357) (layer Edge.Cuts) (width 0.15))
 (gr_arc (start 130.048 62.992) (end 130.683 62.992) (angle -90) (layer Edge.Cuts) (width 0.15))
 (gr_arc (start 130.048 81.788) (end 130.048 82.423) (angle -90) (layer Edge.Cuts) (width 0.15))
 (gr_arc (start 121.412 81.788) (end 120.777 81.788) (angle -90) (layer Edge.Cuts) (width 0.15))
 (gr_arc (start 121.412 62.992) (end 121.412 62.357) (angle -90) (layer Edge.Cuts) (width 0.15))
 (segment (start 124.7925 68.58) (end 121.92 68.58) (width 0.25) (layer F.Cu) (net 11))
 (segment (start 123.73 68.58) (end 121.92 68.58) (width 0.25) (layer B.Cu) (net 11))
 (segment (start 126.6675 68.58) (end 129.54 68.58) (width 0.25) (layer F.Cu) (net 12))
 (segment (start 127.73 68.58) (end 129.54 68.58) (width 0.25) (layer B.Cu) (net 12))
 (segment (start 126.5175 71.12) (end 129.54 71.12) (width 0.25) (layer F.Cu) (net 9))
 (segment (start 127.73 71.12) (end 129.54 71.12) (width 0.25) (layer B.Cu) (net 9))
 (segment (start 124.7925 71.12) (end 121.92 71.12) (width 0.25) (layer F.Cu) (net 10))
 (segment (start 123.73 71.12) (end 121.92 71.12) (width 0.25) (layer B.Cu) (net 10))
 (segment (start 124.7925 63.5) (end 121.92 63.5) (width 0.25) (layer F.Cu) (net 16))
 (segment (start 123.73 63.5) (end 121.92 63.5) (width 0.25) (layer B.Cu) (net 16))
 (segment (start 123.73 63.5) (end 124.63 63.5) (width 0.25) (layer B.Cu) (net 16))
 (segment (start 126.6675 63.5) (end 129.54 63.5) (width 0.25) (layer F.Cu) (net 15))
 (segment (start 126.5175 63.5) (end 129.54 63.5) (width 0.25) (layer F.Cu) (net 15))
 (segment (start 127.73 63.5) (end 129.54 63.5) (width 0.25) (layer B.Cu) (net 15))
 (segment (start 126.6675 66.04) (end 129.54 66.04) (width 0.25) (layer F.Cu) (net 13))
 (segment (start 127.73 66.04) (end 129.54 66.04) (width 0.25) (layer B.Cu) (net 13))
 (segment (start 124.7925 66.04) (end 121.92 66.04) (width 0.25) (layer F.Cu) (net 14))
 (segment (start 123.73 66.04) (end 124.63 66.04) (width 0.25) (layer B.Cu) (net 14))
 (segment (start 123.73 66.04) (end 121.92 66.04) (width 0.25) (layer B.Cu) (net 14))
 (segment (start 126.6675 73.66) (end 129.54 73.66) (width 0.25) (layer F.Cu) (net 8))
 (segment (start 127.73 73.66) (end 129.54 73.66) (width 0.25) (layer B.Cu) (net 8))
 (segment (start 126.6675 76.2) (end 129.54 76.2) (width 0.25) (layer F.Cu) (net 5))
 (segment (start 127.73 76.2) (end 129.54 76.2) (width 0.25) (layer B.Cu) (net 5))
 (segment (start 127.13 78.74) (end 129.54 78.74) (width 0.25) (layer F.Cu) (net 3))
 (segment (start 127.73 78.74) (end 129.54 78.74) (width 0.25) (layer B.Cu) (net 3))
 (segment (start 126.6675 81.28) (end 129.54 81.28) (width 0.25) (layer F.Cu) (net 2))
 (segment (start 127.73 81.28) (end 129.54 81.28) (width 0.25) (layer B.Cu) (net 2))
 (segment (start 124.9425 81.28) (end 121.92 81.28) (width 0.25) (layer F.Cu) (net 1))
 (segment (start 123.73 81.28) (end 121.92 81.28) (width 0.25) (layer B.Cu) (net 1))
 (segment (start 124.7925 78.74) (end 121.92 78.74) (width 0.25) (layer F.Cu) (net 4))
 (segment (start 123.73 78.74) (end 121.92 78.74) (width 0.25) (layer B.Cu) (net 4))
 (segment (start 124.7925 76.2) (end 121.92 76.2) (width 0.25) (layer F.Cu) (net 6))
 (segment (start 123.73 76.2) (end 121.92 76.2) (width 0.25) (layer B.Cu) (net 6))
 (segment (start 124.7925 73.66) (end 121.92 73.66) (width 0.25) (layer F.Cu) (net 7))
 (segment (start 123.73 73.66) (end 121.92 73.66) (width 0.25) (layer B.Cu) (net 7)))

